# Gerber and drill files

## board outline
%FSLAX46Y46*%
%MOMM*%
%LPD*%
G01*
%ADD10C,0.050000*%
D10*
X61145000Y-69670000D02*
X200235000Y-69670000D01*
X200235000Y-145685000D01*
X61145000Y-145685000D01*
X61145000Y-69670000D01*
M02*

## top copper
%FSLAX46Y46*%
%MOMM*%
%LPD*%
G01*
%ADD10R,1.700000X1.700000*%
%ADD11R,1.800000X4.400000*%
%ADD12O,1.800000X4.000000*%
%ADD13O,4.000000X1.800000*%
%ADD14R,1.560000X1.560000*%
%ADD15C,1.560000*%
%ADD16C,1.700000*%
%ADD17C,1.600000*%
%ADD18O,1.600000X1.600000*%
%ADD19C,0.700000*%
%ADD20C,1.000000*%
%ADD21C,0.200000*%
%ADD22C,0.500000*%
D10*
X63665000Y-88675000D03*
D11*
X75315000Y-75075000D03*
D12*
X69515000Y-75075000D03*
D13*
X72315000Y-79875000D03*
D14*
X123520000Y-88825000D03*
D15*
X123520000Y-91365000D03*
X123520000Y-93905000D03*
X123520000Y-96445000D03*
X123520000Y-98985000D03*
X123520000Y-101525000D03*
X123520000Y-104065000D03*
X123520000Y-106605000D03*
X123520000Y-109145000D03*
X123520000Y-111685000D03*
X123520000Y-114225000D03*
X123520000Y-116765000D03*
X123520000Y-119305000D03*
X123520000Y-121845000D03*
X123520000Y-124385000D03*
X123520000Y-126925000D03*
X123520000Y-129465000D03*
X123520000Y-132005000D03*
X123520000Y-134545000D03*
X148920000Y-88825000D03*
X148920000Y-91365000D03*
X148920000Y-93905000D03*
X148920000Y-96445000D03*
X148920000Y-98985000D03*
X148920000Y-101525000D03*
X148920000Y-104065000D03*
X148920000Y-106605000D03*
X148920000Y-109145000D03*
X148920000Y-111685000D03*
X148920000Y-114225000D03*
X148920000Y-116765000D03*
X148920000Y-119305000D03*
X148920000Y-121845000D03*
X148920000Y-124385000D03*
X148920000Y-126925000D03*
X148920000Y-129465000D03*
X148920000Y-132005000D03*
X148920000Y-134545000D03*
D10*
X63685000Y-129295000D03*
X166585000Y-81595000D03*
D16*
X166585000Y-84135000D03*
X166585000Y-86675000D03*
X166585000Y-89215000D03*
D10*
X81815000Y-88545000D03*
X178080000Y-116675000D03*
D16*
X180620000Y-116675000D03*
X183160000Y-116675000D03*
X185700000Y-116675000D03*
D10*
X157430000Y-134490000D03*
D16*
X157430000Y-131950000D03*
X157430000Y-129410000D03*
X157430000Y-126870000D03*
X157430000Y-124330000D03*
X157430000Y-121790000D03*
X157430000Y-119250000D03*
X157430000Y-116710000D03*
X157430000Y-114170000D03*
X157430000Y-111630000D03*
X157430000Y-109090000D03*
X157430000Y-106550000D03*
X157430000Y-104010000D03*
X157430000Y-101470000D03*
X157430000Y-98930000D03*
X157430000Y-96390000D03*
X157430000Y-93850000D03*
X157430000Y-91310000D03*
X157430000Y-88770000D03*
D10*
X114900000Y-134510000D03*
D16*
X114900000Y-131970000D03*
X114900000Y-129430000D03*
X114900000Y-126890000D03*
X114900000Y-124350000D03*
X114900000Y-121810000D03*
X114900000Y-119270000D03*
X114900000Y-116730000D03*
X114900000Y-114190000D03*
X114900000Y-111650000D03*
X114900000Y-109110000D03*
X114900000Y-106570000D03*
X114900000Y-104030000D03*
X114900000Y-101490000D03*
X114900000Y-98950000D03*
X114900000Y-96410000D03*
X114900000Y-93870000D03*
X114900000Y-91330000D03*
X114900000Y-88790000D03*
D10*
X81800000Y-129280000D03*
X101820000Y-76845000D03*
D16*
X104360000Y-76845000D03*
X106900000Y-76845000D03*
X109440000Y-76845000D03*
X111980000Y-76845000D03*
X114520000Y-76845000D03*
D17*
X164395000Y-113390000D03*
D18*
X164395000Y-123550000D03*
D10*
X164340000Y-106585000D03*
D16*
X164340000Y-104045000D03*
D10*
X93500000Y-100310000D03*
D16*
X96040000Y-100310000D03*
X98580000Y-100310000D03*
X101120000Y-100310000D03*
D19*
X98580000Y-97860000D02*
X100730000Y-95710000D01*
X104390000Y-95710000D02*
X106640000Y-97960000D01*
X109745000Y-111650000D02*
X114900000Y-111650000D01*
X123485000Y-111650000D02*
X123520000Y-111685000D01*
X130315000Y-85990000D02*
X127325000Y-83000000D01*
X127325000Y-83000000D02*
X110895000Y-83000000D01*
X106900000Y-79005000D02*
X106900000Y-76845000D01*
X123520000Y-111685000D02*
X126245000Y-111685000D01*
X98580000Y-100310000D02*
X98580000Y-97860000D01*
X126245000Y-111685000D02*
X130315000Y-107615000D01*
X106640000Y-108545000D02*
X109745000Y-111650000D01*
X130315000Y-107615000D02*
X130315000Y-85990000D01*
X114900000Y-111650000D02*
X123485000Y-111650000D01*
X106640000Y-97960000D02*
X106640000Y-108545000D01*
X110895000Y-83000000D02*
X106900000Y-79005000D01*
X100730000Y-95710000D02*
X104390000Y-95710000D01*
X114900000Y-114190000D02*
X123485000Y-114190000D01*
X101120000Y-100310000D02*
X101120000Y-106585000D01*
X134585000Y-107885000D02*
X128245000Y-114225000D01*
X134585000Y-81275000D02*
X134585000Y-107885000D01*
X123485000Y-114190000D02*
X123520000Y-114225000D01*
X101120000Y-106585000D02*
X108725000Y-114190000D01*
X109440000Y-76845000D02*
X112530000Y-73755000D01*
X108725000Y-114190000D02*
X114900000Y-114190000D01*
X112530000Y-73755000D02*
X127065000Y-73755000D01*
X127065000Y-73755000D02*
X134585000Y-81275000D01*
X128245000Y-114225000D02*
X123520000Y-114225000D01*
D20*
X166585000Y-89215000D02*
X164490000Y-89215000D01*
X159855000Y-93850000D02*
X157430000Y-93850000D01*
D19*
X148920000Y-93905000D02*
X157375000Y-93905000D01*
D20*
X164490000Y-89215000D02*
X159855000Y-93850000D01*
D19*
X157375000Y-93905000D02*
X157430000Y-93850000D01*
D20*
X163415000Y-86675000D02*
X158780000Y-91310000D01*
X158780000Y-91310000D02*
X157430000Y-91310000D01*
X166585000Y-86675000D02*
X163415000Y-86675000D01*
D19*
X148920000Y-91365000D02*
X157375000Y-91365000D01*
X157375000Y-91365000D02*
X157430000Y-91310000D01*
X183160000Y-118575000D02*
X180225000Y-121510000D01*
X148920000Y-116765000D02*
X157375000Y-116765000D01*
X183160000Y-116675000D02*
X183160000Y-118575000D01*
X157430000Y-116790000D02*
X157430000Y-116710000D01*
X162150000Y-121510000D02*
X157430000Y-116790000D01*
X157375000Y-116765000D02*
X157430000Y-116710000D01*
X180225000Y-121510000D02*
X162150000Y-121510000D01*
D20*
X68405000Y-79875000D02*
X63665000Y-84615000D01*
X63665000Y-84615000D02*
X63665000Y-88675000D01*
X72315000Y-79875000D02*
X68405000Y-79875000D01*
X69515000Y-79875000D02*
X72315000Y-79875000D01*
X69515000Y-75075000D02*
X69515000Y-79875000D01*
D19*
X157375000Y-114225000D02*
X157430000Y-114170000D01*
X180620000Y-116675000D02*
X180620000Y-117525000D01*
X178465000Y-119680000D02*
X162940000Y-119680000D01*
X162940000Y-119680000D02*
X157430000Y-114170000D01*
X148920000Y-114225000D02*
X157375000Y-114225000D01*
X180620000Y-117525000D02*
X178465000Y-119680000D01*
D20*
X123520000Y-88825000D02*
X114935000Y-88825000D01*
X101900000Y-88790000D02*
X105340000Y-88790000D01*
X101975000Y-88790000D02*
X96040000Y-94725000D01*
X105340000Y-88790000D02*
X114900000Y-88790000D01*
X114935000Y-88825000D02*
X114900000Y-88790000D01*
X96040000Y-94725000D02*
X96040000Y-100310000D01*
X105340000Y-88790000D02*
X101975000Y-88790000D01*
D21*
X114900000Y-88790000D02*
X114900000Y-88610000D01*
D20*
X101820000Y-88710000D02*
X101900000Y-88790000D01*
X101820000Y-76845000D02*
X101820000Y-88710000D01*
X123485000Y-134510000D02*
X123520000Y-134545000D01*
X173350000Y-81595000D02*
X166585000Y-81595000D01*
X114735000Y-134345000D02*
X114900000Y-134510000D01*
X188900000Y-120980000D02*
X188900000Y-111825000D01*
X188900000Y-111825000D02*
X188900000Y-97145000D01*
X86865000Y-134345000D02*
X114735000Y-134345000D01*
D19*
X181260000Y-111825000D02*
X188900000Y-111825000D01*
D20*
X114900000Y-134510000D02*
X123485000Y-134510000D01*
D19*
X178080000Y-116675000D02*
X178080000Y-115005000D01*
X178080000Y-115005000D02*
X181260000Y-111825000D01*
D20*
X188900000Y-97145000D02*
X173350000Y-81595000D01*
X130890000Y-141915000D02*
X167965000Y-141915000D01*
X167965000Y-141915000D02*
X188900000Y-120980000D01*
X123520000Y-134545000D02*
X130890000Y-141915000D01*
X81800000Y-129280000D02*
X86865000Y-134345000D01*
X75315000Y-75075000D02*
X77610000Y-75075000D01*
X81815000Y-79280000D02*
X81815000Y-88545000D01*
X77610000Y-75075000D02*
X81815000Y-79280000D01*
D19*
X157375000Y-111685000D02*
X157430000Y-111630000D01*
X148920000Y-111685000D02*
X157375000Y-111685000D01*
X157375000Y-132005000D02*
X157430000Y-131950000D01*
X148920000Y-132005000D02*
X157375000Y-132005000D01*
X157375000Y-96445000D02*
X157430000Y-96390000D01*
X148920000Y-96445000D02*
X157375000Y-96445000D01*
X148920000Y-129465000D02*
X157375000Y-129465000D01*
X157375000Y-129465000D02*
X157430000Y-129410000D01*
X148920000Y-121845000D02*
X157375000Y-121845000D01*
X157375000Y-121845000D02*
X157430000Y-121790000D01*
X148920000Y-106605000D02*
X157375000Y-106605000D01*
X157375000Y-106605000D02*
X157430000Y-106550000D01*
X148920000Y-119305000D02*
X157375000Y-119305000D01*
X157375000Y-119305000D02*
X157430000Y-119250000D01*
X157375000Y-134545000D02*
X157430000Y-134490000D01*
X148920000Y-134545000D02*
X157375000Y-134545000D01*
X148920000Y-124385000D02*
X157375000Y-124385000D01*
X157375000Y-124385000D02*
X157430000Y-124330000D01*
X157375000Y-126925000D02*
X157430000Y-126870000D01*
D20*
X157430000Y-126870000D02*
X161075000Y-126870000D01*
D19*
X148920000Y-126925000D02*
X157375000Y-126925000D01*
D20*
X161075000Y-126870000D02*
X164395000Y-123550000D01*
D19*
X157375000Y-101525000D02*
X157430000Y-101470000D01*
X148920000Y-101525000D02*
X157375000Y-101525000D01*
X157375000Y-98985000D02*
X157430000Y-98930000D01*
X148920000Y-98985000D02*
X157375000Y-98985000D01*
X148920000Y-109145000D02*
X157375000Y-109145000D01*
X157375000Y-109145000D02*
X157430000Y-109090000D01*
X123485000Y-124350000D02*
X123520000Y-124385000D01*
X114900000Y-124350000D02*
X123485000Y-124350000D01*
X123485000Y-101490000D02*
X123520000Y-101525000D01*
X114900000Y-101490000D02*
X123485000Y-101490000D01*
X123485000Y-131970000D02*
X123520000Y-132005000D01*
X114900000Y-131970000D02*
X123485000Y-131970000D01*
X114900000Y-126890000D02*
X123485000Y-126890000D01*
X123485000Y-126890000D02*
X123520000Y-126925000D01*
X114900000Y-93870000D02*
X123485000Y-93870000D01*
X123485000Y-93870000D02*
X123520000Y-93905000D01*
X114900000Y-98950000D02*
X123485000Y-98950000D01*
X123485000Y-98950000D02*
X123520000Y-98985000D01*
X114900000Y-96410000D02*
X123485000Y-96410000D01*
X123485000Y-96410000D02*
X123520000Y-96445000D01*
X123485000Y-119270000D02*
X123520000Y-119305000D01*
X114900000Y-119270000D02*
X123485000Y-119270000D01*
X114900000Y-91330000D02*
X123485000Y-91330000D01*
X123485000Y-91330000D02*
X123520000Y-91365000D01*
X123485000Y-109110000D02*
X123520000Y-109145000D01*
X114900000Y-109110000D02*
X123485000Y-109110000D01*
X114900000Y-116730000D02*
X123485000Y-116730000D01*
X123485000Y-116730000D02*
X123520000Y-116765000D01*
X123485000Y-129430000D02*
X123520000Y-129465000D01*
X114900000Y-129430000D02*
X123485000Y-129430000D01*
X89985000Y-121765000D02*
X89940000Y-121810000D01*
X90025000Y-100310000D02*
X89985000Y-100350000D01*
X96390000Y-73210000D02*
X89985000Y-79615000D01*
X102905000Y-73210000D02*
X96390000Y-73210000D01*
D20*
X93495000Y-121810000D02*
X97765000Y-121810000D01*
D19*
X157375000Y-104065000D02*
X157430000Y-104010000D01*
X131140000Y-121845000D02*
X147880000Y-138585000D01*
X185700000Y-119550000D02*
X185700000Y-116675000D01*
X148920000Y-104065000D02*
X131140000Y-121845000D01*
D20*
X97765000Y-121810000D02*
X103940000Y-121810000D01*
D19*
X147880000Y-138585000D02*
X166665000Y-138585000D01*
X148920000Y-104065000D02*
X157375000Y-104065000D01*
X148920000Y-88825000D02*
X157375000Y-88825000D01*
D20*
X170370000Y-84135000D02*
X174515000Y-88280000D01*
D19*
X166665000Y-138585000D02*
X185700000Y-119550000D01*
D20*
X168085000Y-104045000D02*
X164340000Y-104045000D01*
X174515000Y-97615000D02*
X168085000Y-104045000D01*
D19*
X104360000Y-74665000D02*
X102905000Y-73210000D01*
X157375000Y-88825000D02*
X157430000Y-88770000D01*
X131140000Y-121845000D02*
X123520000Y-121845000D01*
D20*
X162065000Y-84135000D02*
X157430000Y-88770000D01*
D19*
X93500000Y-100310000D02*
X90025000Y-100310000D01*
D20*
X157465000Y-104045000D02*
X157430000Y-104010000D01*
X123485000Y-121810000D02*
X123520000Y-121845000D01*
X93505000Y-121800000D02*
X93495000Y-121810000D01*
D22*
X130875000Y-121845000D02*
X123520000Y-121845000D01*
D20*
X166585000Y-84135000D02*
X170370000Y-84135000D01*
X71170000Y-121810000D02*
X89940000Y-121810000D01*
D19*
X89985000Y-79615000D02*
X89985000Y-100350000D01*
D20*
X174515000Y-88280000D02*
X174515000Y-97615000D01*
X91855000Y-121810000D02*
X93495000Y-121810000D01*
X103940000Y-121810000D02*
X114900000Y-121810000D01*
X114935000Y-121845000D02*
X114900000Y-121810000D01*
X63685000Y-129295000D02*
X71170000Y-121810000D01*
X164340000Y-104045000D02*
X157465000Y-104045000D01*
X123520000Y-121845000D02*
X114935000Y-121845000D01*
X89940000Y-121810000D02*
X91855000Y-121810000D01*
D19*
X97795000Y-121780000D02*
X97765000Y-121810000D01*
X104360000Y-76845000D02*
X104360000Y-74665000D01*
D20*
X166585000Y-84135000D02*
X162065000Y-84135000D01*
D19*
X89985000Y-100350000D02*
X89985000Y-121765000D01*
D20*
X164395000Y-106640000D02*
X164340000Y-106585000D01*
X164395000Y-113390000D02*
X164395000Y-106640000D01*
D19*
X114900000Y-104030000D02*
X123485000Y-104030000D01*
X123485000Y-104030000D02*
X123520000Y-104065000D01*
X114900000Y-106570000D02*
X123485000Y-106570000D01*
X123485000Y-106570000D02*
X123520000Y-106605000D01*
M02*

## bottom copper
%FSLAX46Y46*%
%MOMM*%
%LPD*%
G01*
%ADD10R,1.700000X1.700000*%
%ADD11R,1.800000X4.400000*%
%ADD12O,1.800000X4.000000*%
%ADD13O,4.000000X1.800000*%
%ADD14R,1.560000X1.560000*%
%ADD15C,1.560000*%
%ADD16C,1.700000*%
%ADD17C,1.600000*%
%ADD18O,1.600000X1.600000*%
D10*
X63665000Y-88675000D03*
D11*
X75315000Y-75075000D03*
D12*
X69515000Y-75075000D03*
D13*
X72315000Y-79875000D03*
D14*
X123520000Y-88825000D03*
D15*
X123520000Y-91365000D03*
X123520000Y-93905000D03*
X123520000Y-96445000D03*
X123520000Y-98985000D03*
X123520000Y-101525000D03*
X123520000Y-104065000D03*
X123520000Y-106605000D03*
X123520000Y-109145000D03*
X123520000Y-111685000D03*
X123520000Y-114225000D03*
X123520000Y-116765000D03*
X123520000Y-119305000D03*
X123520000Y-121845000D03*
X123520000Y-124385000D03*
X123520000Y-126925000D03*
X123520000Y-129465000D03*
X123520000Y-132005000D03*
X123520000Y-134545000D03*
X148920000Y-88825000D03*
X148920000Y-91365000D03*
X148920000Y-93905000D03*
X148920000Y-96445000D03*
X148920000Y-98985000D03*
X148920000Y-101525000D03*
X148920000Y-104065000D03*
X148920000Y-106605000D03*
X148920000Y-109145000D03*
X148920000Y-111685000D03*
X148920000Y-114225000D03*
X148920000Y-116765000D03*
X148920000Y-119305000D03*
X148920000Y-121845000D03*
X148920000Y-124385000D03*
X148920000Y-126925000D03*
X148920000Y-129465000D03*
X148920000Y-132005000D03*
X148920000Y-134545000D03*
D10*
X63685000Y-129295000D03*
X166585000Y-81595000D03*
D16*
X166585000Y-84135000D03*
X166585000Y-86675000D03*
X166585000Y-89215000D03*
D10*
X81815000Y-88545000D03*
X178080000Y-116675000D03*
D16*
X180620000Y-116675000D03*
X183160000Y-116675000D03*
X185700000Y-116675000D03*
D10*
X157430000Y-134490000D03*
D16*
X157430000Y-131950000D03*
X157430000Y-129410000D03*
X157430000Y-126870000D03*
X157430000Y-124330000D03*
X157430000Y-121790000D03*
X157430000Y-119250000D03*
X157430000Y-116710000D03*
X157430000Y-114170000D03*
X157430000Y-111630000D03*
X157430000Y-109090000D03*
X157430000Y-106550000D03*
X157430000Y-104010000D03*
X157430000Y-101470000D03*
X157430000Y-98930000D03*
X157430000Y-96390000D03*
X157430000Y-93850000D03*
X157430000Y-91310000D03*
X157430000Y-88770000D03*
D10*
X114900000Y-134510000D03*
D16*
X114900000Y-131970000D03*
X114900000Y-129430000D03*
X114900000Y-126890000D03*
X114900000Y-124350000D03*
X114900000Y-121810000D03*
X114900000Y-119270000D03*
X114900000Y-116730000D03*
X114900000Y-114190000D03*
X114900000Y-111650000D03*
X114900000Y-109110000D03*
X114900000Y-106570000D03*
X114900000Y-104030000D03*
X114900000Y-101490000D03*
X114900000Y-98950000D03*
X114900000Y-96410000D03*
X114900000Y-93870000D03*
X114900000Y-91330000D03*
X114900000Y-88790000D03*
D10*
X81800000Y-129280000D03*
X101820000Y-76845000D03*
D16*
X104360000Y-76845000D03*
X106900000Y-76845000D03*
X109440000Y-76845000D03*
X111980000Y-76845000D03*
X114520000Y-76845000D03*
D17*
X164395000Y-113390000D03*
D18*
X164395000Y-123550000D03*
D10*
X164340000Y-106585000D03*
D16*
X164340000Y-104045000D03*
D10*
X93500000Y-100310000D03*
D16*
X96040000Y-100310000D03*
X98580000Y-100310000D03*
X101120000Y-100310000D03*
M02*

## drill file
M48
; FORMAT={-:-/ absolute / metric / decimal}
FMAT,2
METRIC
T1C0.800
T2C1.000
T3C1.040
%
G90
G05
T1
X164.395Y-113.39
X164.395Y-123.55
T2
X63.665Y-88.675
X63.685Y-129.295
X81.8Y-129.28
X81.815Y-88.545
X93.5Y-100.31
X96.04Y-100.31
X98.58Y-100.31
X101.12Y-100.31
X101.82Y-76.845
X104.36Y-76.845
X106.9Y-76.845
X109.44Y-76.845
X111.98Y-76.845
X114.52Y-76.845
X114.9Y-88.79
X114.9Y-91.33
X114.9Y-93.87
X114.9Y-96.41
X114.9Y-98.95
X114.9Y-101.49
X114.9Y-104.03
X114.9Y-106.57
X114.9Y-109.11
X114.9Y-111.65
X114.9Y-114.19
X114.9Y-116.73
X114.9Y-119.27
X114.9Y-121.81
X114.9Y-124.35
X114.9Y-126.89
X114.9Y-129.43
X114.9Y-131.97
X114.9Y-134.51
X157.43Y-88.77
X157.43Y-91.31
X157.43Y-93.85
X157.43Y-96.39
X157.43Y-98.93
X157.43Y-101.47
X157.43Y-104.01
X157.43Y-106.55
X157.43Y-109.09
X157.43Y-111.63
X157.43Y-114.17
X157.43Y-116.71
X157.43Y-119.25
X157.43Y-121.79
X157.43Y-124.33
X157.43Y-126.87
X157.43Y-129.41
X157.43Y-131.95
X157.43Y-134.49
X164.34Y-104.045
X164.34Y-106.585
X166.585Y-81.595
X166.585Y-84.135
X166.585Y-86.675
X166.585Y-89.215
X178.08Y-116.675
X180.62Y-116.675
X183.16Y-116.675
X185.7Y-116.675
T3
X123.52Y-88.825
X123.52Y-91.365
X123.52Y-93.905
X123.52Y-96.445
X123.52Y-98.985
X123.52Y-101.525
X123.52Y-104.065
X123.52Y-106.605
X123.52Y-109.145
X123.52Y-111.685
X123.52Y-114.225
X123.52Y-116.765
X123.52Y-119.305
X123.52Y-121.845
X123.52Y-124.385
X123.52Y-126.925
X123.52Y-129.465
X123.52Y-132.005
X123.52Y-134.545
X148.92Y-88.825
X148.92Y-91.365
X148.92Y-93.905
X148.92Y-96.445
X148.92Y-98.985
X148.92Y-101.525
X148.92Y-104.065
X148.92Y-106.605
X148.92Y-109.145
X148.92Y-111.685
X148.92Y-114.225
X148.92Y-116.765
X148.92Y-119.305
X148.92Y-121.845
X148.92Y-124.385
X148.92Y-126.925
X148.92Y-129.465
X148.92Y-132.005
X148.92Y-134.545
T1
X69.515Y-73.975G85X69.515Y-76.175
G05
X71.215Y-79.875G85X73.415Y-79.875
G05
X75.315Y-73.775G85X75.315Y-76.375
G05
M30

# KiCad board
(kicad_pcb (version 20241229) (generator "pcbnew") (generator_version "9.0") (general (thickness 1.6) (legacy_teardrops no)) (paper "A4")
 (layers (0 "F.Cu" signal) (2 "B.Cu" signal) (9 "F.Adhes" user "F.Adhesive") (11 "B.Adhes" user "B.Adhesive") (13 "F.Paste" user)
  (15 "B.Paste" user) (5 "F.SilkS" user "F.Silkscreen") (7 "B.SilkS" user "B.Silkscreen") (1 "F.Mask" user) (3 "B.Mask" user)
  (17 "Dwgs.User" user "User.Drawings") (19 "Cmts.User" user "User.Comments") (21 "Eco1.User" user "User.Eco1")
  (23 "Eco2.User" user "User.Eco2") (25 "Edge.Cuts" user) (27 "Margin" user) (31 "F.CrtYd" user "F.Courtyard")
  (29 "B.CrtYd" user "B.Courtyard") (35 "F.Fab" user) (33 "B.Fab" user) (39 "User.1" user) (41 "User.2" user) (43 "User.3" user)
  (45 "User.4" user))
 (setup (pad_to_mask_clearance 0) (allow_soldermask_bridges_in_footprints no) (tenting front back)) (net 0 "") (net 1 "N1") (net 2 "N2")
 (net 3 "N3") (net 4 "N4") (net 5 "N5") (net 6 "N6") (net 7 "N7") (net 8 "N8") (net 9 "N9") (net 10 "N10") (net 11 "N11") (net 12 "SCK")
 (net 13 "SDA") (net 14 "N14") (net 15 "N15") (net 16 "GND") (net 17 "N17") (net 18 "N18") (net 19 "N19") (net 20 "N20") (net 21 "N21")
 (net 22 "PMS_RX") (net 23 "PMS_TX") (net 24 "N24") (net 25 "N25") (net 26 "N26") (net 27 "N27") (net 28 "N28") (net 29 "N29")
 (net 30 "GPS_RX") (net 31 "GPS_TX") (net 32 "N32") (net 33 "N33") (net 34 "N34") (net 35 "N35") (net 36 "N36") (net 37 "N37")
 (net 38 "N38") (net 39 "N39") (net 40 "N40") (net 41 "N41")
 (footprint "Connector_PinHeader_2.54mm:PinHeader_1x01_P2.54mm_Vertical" (layer "F.Cu") (at 63.665 88.675)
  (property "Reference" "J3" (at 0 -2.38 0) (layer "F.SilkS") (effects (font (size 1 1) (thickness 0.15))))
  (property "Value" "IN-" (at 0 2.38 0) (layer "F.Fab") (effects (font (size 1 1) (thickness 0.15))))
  (pad "1" thru_hole rect (at 0 0) (size 1.7 1.7) (drill 1) (layers "*.Cu" "*.Mask") (remove_unused_layers no) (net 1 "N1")))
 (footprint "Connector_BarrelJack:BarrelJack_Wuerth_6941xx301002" (layer "F.Cu") (at 75.315 75.075 -90)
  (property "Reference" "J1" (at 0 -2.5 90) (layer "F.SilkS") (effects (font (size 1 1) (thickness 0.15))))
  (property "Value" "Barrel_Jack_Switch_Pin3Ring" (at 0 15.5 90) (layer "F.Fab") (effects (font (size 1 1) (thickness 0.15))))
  (pad "1" thru_hole rect (at 0 0 270) (size 4.4 1.8) (drill oval 3.4 0.8) (layers "*.Cu" "*.Mask") (remove_unused_layers no) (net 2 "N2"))
  (pad "2" thru_hole oval (at 0 5.8 270) (size 4 1.8) (drill oval 3 0.8) (layers "*.Cu" "*.Mask") (remove_unused_layers no) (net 1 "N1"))
  (pad "3" thru_hole oval (at 4.8 3) (size 4 1.8) (drill oval 3 0.8) (layers "*.Cu" "*.Mask") (remove_unused_layers no) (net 1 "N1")))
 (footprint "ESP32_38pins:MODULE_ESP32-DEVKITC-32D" (layer "F.Cu") (at 136.22 108.585)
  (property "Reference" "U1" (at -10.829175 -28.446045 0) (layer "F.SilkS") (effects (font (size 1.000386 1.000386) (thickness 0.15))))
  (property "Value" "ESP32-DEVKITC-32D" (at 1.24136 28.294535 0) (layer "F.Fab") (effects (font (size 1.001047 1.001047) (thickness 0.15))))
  (pad "J2-1" thru_hole rect (at -12.7 -19.76) (size 1.56 1.56) (drill 1.04) (layers "*.Cu" "*.Mask") (remove_unused_layers no) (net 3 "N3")
   (solder_mask_margin 0.102))
  (pad "J2-2" thru_hole circle (at -12.7 -17.22) (size 1.56 1.56) (drill 1.04) (layers "*.Cu" "*.Mask") (remove_unused_layers no)
   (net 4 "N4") (solder_mask_margin 0.102))
  (pad "J2-3" thru_hole circle (at -12.7 -14.68) (size 1.56 1.56) (drill 1.04) (layers "*.Cu" "*.Mask") (remove_unused_layers no)
   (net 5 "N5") (solder_mask_margin 0.102))
  (pad "J2-4" thru_hole circle (at -12.7 -12.14) (size 1.56 1.56) (drill 1.04) (layers "*.Cu" "*.Mask") (remove_unused_layers no)
   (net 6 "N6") (solder_mask_margin 0.102))
  (pad "J2-5" thru_hole circle (at -12.7 -9.6) (size 1.56 1.56) (drill 1.04) (layers "*.Cu" "*.Mask") (remove_unused_layers no) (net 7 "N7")
   (solder_mask_margin 0.102))
  (pad "J2-6" thru_hole circle (at -12.7 -7.06) (size 1.56 1.56) (drill 1.04) (layers "*.Cu" "*.Mask") (remove_unused_layers no)
   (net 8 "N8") (solder_mask_margin 0.102))
  (pad "J2-7" thru_hole circle (at -12.7 -4.52) (size 1.56 1.56) (drill 1.04) (layers "*.Cu" "*.Mask") (remove_unused_layers no)
   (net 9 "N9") (solder_mask_margin 0.102))
  (pad "J2-8" thru_hole circle (at -12.7 -1.98) (size 1.56 1.56) (drill 1.04) (layers "*.Cu" "*.Mask") (remove_unused_layers no)
   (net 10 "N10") (solder_mask_margin 0.102))
  (pad "J2-9" thru_hole circle (at -12.7 0.56) (size 1.56 1.56) (drill 1.04) (layers "*.Cu" "*.Mask") (remove_unused_layers no)
   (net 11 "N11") (solder_mask_margin 0.102))
  (pad "J2-10" thru_hole circle (at -12.7 3.1) (size 1.56 1.56) (drill 1.04) (layers "*.Cu" "*.Mask") (remove_unused_layers no)
   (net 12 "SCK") (solder_mask_margin 0.102))
  (pad "J2-11" thru_hole circle (at -12.7 5.64) (size 1.56 1.56) (drill 1.04) (layers "*.Cu" "*.Mask") (remove_unused_layers no)
   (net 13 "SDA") (solder_mask_margin 0.102))
  (pad "J2-12" thru_hole circle (at -12.7 8.18) (size 1.56 1.56) (drill 1.04) (layers "*.Cu" "*.Mask") (remove_unused_layers no)
   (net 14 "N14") (solder_mask_margin 0.102))
  (pad "J2-13" thru_hole circle (at -12.7 10.72) (size 1.56 1.56) (drill 1.04) (layers "*.Cu" "*.Mask") (remove_unused_layers no)
   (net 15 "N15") (solder_mask_margin 0.102))
  (pad "J2-14" thru_hole circle (at -12.7 13.26) (size 1.56 1.56) (drill 1.04) (layers "*.Cu" "*.Mask") (remove_unused_layers no)
   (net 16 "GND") (solder_mask_margin 0.102))
  (pad "J2-15" thru_hole circle (at -12.7 15.8) (size 1.56 1.56) (drill 1.04) (layers "*.Cu" "*.Mask") (remove_unused_layers no)
   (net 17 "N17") (solder_mask_margin 0.102))
  (pad "J2-16" thru_hole circle (at -12.7 18.34) (size 1.56 1.56) (drill 1.04) (layers "*.Cu" "*.Mask") (remove_unused_layers no)
   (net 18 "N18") (solder_mask_margin 0.102))
  (pad "J2-17" thru_hole circle (at -12.7 20.88) (size 1.56 1.56) (drill 1.04) (layers "*.Cu" "*.Mask") (remove_unused_layers no)
   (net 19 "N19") (solder_mask_margin 0.102))
  (pad "J2-18" thru_hole circle (at -12.7 23.42) (size 1.56 1.56) (drill 1.04) (layers "*.Cu" "*.Mask") (remove_unused_layers no)
   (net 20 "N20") (solder_mask_margin 0.102))
  (pad "J2-19" thru_hole circle (at -12.7 25.96) (size 1.56 1.56) (drill 1.04) (layers "*.Cu" "*.Mask") (remove_unused_layers no)
   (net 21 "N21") (solder_mask_margin 0.102))
  (pad "J3-1" thru_hole circle (at 12.7 -19.76) (size 1.56 1.56) (drill 1.04) (layers "*.Cu" "*.Mask") (remove_unused_layers no)
   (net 16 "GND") (solder_mask_margin 0.102))
  (pad "J3-2" thru_hole circle (at 12.7 -17.22) (size 1.56 1.56) (drill 1.04) (layers "*.Cu" "*.Mask") (remove_unused_layers no)
   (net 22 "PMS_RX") (solder_mask_margin 0.102))
  (pad "J3-3" thru_hole circle (at 12.7 -14.68) (size 1.56 1.56) (drill 1.04) (layers "*.Cu" "*.Mask") (remove_unused_layers no)
   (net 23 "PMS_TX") (solder_mask_margin 0.102))
  (pad "J3-4" thru_hole circle (at 12.7 -12.14) (size 1.56 1.56) (drill 1.04) (layers "*.Cu" "*.Mask") (remove_unused_layers no)
   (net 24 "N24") (solder_mask_margin 0.102))
  (pad "J3-5" thru_hole circle (at 12.7 -9.6) (size 1.56 1.56) (drill 1.04) (layers "*.Cu" "*.Mask") (remove_unused_layers no)
   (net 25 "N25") (solder_mask_margin 0.102))
  (pad "J3-6" thru_hole circle (at 12.7 -7.06) (size 1.56 1.56) (drill 1.04) (layers "*.Cu" "*.Mask") (remove_unused_layers no)
   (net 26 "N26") (solder_mask_margin 0.102))
  (pad "J3-7" thru_hole circle (at 12.7 -4.52) (size 1.56 1.56) (drill 1.04) (layers "*.Cu" "*.Mask") (remove_unused_layers no)
   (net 16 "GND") (solder_mask_margin 0.102))
  (pad "J3-8" thru_hole circle (at 12.7 -1.98) (size 1.56 1.56) (drill 1.04) (layers "*.Cu" "*.Mask") (remove_unused_layers no)
   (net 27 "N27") (solder_mask_margin 0.102))
  (pad "J3-9" thru_hole circle (at 12.7 0.56) (size 1.56 1.56) (drill 1.04) (layers "*.Cu" "*.Mask") (remove_unused_layers no)
   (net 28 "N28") (solder_mask_margin 0.102))
  (pad "J3-10" thru_hole circle (at 12.7 3.1) (size 1.56 1.56) (drill 1.04) (layers "*.Cu" "*.Mask") (remove_unused_layers no)
   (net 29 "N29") (solder_mask_margin 0.102))
  (pad "J3-11" thru_hole circle (at 12.7 5.64) (size 1.56 1.56) (drill 1.04) (layers "*.Cu" "*.Mask") (remove_unused_layers no)
   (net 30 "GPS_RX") (solder_mask_margin 0.102))
  (pad "J3-12" thru_hole circle (at 12.7 8.18) (size 1.56 1.56) (drill 1.04) (layers "*.Cu" "*.Mask") (remove_unused_layers no)
   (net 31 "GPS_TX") (solder_mask_margin 0.102))
  (pad "J3-13" thru_hole circle (at 12.7 10.72) (size 1.56 1.56) (drill 1.04) (layers "*.Cu" "*.Mask") (remove_unused_layers no)
   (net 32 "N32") (solder_mask_margin 0.102))
  (pad "J3-14" thru_hole circle (at 12.7 13.26) (size 1.56 1.56) (drill 1.04) (layers "*.Cu" "*.Mask") (remove_unused_layers no)
   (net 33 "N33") (solder_mask_margin 0.102))
  (pad "J3-15" thru_hole circle (at 12.7 15.8) (size 1.56 1.56) (drill 1.04) (layers "*.Cu" "*.Mask") (remove_unused_layers no)
   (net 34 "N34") (solder_mask_margin 0.102))
  (pad "J3-16" thru_hole circle (at 12.7 18.34) (size 1.56 1.56) (drill 1.04) (layers "*.Cu" "*.Mask") (remove_unused_layers no)
   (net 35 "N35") (solder_mask_margin 0.102))
  (pad "J3-17" thru_hole circle (at 12.7 20.88) (size 1.56 1.56) (drill 1.04) (layers "*.Cu" "*.Mask") (remove_unused_layers no)
   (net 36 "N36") (solder_mask_margin 0.102))
  (pad "J3-18" thru_hole circle (at 12.7 23.42) (size 1.56 1.56) (drill 1.04) (layers "*.Cu" "*.Mask") (remove_unused_layers no)
   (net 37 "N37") (solder_mask_margin 0.102))
  (pad "J3-19" thru_hole circle (at 12.7 25.96) (size 1.56 1.56) (drill 1.04) (layers "*.Cu" "*.Mask") (remove_unused_layers no)
   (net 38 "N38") (solder_mask_margin 0.102)))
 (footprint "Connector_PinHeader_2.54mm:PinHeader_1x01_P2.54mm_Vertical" (layer "F.Cu") (at 63.685 129.295)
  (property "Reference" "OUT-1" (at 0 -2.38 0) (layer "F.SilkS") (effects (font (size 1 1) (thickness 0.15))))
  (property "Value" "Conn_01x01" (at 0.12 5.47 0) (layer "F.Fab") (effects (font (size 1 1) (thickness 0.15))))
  (pad "1" thru_hole rect (at 0 0) (size 1.7 1.7) (drill 1) (layers "*.Cu" "*.Mask") (remove_unused_layers no) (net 16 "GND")))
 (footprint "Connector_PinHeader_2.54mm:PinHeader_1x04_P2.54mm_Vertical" (layer "F.Cu") (at 166.585 81.595)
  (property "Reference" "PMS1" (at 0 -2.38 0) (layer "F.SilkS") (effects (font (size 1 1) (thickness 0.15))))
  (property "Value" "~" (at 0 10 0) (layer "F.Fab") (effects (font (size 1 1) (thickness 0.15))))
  (pad "1" thru_hole rect (at 0 0) (size 1.7 1.7) (drill 1) (layers "*.Cu" "*.Mask") (remove_unused_layers no) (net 21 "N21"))
  (pad "2" thru_hole circle (at 0 2.54) (size 1.7 1.7) (drill 1) (layers "*.Cu" "*.Mask") (remove_unused_layers no) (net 16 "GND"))
  (pad "3" thru_hole circle (at 0 5.08) (size 1.7 1.7) (drill 1) (layers "*.Cu" "*.Mask") (remove_unused_layers no) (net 22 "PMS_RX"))
  (pad "4" thru_hole circle (at 0 7.62) (size 1.7 1.7) (drill 1) (layers "*.Cu" "*.Mask") (remove_unused_layers no) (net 23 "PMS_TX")))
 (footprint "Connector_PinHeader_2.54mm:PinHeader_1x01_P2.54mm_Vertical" (layer "F.Cu") (at 81.815 88.545)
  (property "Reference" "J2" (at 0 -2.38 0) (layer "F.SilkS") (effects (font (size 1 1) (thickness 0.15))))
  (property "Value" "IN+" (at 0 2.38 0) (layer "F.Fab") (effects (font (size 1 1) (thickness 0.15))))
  (pad "1" thru_hole rect (at 0 0) (size 1.7 1.7) (drill 1) (layers "*.Cu" "*.Mask") (remove_unused_layers no) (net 2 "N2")))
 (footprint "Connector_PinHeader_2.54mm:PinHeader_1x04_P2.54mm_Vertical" (layer "F.Cu") (at 178.08 116.675 90)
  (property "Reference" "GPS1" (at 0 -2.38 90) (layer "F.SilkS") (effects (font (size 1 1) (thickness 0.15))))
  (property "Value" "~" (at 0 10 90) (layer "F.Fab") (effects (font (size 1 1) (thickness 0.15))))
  (pad "1" thru_hole rect (at 0 0 90) (size 1.7 1.7) (drill 1) (layers "*.Cu" "*.Mask") (remove_unused_layers no) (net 21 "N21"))
  (pad "2" thru_hole circle (at 0 2.54 90) (size 1.7 1.7) (drill 1) (layers "*.Cu" "*.Mask") (remove_unused_layers no) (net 30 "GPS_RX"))
  (pad "3" thru_hole circle (at 0 5.08 90) (size 1.7 1.7) (drill 1) (layers "*.Cu" "*.Mask") (remove_unused_layers no) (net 31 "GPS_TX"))
  (pad "4" thru_hole circle (at 0 7.62 90) (size 1.7 1.7) (drill 1) (layers "*.Cu" "*.Mask") (remove_unused_layers no) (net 16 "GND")))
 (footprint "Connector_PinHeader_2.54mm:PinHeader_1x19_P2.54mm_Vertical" (layer "F.Cu") (at 157.43 134.49 180)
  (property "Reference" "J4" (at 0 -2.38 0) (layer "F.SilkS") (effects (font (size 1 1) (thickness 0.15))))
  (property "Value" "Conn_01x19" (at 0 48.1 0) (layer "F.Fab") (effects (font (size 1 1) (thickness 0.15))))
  (pad "1" thru_hole rect (at 0 0 180) (size 1.7 1.7) (drill 1) (layers "*.Cu" "*.Mask") (remove_unused_layers no) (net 38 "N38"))
  (pad "2" thru_hole circle (at 0 2.54 180) (size 1.7 1.7) (drill 1) (layers "*.Cu" "*.Mask") (remove_unused_layers no) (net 37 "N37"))
  (pad "3" thru_hole circle (at 0 5.08 180) (size 1.7 1.7) (drill 1) (layers "*.Cu" "*.Mask") (remove_unused_layers no) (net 36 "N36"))
  (pad "4" thru_hole circle (at 0 7.62 180) (size 1.7 1.7) (drill 1) (layers "*.Cu" "*.Mask") (remove_unused_layers no) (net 35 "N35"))
  (pad "5" thru_hole circle (at 0 10.16 180) (size 1.7 1.7) (drill 1) (layers "*.Cu" "*.Mask") (remove_unused_layers no) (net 34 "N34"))
  (pad "6" thru_hole circle (at 0 12.7 180) (size 1.7 1.7) (drill 1) (layers "*.Cu" "*.Mask") (remove_unused_layers no) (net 33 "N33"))
  (pad "7" thru_hole circle (at 0 15.24 180) (size 1.7 1.7) (drill 1) (layers "*.Cu" "*.Mask") (remove_unused_layers no) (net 32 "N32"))
  (pad "8" thru_hole circle (at 0 17.78 180) (size 1.7 1.7) (drill 1) (layers "*.Cu" "*.Mask") (remove_unused_layers no) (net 31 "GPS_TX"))
  (pad "9" thru_hole circle (at 0 20.32 180) (size 1.7 1.7) (drill 1) (layers "*.Cu" "*.Mask") (remove_unused_layers no) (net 30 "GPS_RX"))
  (pad "10" thru_hole circle (at 0 22.86 180) (size 1.7 1.7) (drill 1) (layers "*.Cu" "*.Mask") (remove_unused_layers no) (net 29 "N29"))
  (pad "11" thru_hole circle (at 0 25.4 180) (size 1.7 1.7) (drill 1) (layers "*.Cu" "*.Mask") (remove_unused_layers no) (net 28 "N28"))
  (pad "12" thru_hole circle (at 0 27.94 180) (size 1.7 1.7) (drill 1) (layers "*.Cu" "*.Mask") (remove_unused_layers no) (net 27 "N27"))
  (pad "13" thru_hole circle (at 0 30.48 180) (size 1.7 1.7) (drill 1) (layers "*.Cu" "*.Mask") (remove_unused_layers no) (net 16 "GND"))
  (pad "14" thru_hole circle (at 0 33.02 180) (size 1.7 1.7) (drill 1) (layers "*.Cu" "*.Mask") (remove_unused_layers no) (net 26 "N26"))
  (pad "15" thru_hole circle (at 0 35.56 180) (size 1.7 1.7) (drill 1) (layers "*.Cu" "*.Mask") (remove_unused_layers no) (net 25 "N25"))
  (pad "16" thru_hole circle (at 0 38.1 180) (size 1.7 1.7) (drill 1) (layers "*.Cu" "*.Mask") (remove_unused_layers no) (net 24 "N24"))
  (pad "17" thru_hole circle (at 0 40.64 180) (size 1.7 1.7) (drill 1) (layers "*.Cu" "*.Mask") (remove_unused_layers no) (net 23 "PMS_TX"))
  (pad "18" thru_hole circle (at 0 43.18 180) (size 1.7 1.7) (drill 1) (layers "*.Cu" "*.Mask") (remove_unused_layers no) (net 22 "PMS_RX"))
  (pad "19" thru_hole circle (at 0 45.72 180) (size 1.7 1.7) (drill 1) (layers "*.Cu" "*.Mask") (remove_unused_layers no) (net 16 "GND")))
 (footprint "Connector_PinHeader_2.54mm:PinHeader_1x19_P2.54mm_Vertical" (layer "F.Cu") (at 114.9 134.51 180)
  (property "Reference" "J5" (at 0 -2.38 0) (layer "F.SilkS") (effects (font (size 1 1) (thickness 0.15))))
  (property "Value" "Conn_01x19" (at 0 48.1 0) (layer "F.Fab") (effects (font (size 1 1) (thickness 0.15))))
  (pad "1" thru_hole rect (at 0 0 180) (size 1.7 1.7) (drill 1) (layers "*.Cu" "*.Mask") (remove_unused_layers no) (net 21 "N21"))
  (pad "2" thru_hole circle (at 0 2.54 180) (size 1.7 1.7) (drill 1) (layers "*.Cu" "*.Mask") (remove_unused_layers no) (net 20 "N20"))
  (pad "3" thru_hole circle (at 0 5.08 180) (size 1.7 1.7) (drill 1) (layers "*.Cu" "*.Mask") (remove_unused_layers no) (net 19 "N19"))
  (pad "4" thru_hole circle (at 0 7.62 180) (size 1.7 1.7) (drill 1) (layers "*.Cu" "*.Mask") (remove_unused_layers no) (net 18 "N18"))
  (pad "5" thru_hole circle (at 0 10.16 180) (size 1.7 1.7) (drill 1) (layers "*.Cu" "*.Mask") (remove_unused_layers no) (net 17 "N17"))
  (pad "6" thru_hole circle (at 0 12.7 180) (size 1.7 1.7) (drill 1) (layers "*.Cu" "*.Mask") (remove_unused_layers no) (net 16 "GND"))
  (pad "7" thru_hole circle (at 0 15.24 180) (size 1.7 1.7) (drill 1) (layers "*.Cu" "*.Mask") (remove_unused_layers no) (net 15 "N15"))
  (pad "8" thru_hole circle (at 0 17.78 180) (size 1.7 1.7) (drill 1) (layers "*.Cu" "*.Mask") (remove_unused_layers no) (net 14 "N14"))
  (pad "9" thru_hole circle (at 0 20.32 180) (size 1.7 1.7) (drill 1) (layers "*.Cu" "*.Mask") (remove_unused_layers no) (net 13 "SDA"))
  (pad "10" thru_hole circle (at 0 22.86 180) (size 1.7 1.7) (drill 1) (layers "*.Cu" "*.Mask") (remove_unused_layers no) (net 12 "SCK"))
  (pad "11" thru_hole circle (at 0 25.4 180) (size 1.7 1.7) (drill 1) (layers "*.Cu" "*.Mask") (remove_unused_layers no) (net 11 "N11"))
  (pad "12" thru_hole circle (at 0 27.94 180) (size 1.7 1.7) (drill 1) (layers "*.Cu" "*.Mask") (remove_unused_layers no) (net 10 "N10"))
  (pad "13" thru_hole circle (at 0 30.48 180) (size 1.7 1.7) (drill 1) (layers "*.Cu" "*.Mask") (remove_unused_layers no) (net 9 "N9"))
  (pad "14" thru_hole circle (at 0 33.02 180) (size 1.7 1.7) (drill 1) (layers "*.Cu" "*.Mask") (remove_unused_layers no) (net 8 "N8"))
  (pad "15" thru_hole circle (at 0 35.56 180) (size 1.7 1.7) (drill 1) (layers "*.Cu" "*.Mask") (remove_unused_layers no) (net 7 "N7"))
  (pad "16" thru_hole circle (at 0 38.1 180) (size 1.7 1.7) (drill 1) (layers "*.Cu" "*.Mask") (remove_unused_layers no) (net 6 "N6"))
  (pad "17" thru_hole circle (at 0 40.64 180) (size 1.7 1.7) (drill 1) (layers "*.Cu" "*.Mask") (remove_unused_layers no) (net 5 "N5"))
  (pad "18" thru_hole circle (at 0 43.18 180) (size 1.7 1.7) (drill 1) (layers "*.Cu" "*.Mask") (remove_unused_layers no) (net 4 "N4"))
  (pad "19" thru_hole circle (at 0 45.72 180) (size 1.7 1.7) (drill 1) (layers "*.Cu" "*.Mask") (remove_unused_layers no) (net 3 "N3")))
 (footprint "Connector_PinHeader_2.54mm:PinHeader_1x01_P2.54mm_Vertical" (layer "F.Cu") (at 81.8 129.28)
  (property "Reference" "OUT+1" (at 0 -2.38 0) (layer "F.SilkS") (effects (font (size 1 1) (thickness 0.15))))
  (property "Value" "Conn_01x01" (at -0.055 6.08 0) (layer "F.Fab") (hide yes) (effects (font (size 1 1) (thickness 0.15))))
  (pad "1" thru_hole rect (at 0 0) (size 1.7 1.7) (drill 1) (layers "*.Cu" "*.Mask") (remove_unused_layers no) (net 21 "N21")))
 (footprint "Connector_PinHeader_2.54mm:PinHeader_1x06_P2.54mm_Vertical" (layer "F.Cu") (at 101.82 76.845 90)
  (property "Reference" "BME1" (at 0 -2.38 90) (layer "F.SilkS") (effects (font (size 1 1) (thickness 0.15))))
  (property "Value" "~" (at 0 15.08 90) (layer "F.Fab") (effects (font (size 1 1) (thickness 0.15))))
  (pad "1" thru_hole rect (at 0 0 90) (size 1.7 1.7) (drill 1) (layers "*.Cu" "*.Mask") (remove_unused_layers no) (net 3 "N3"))
  (pad "2" thru_hole circle (at 0 2.54 90) (size 1.7 1.7) (drill 1) (layers "*.Cu" "*.Mask") (remove_unused_layers no) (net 16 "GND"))
  (pad "3" thru_hole circle (at 0 5.08 90) (size 1.7 1.7) (drill 1) (layers "*.Cu" "*.Mask") (remove_unused_layers no) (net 12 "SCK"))
  (pad "4" thru_hole circle (at 0 7.62 90) (size 1.7 1.7) (drill 1) (layers "*.Cu" "*.Mask") (remove_unused_layers no) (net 13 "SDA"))
  (pad "5" thru_hole circle (at 0 10.16 90) (size 1.7 1.7) (drill 1) (layers "*.Cu" "*.Mask") (remove_unused_layers no) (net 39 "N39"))
  (pad "6" thru_hole circle (at 0 12.7 90) (size 1.7 1.7) (drill 1) (layers "*.Cu" "*.Mask") (remove_unused_layers no) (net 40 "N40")))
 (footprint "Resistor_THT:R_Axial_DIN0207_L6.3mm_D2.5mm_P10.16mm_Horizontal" (layer "F.Cu") (at 164.395 113.39 -90)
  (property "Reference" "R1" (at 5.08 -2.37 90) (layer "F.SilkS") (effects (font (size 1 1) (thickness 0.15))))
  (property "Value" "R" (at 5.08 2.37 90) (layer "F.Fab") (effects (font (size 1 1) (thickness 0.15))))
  (pad "1" thru_hole circle (at 0 0 270) (size 1.6 1.6) (drill 0.8) (layers "*.Cu" "*.Mask") (remove_unused_layers no) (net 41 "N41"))
  (pad "2" thru_hole oval (at 10.16 0 270) (size 1.6 1.6) (drill 0.8) (layers "*.Cu" "*.Mask") (remove_unused_layers no) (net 35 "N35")))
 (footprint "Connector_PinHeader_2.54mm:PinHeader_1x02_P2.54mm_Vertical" (layer "F.Cu") (at 164.34 106.585 180)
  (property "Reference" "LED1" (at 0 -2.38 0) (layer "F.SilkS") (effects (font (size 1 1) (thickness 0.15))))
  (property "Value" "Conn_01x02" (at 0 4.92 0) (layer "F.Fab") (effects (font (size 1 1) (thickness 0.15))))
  (pad "1" thru_hole rect (at 0 0 180) (size 1.7 1.7) (drill 1) (layers "*.Cu" "*.Mask") (remove_unused_layers no) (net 41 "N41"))
  (pad "2" thru_hole circle (at 0 2.54 180) (size 1.7 1.7) (drill 1) (layers "*.Cu" "*.Mask") (remove_unused_layers no) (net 16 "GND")))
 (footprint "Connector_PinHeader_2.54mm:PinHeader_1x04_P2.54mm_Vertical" (layer "F.Cu") (at 93.5 100.31 90)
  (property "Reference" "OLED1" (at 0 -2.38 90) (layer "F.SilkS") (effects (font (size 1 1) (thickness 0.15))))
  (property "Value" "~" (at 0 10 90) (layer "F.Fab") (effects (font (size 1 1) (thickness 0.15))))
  (pad "1" thru_hole rect (at 0 0 90) (size 1.7 1.7) (drill 1) (layers "*.Cu" "*.Mask") (remove_unused_layers no) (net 16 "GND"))
  (pad "2" thru_hole circle (at 0 2.54 90) (size 1.7 1.7) (drill 1) (layers "*.Cu" "*.Mask") (remove_unused_layers no) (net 3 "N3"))
  (pad "3" thru_hole circle (at 0 5.08 90) (size 1.7 1.7) (drill 1) (layers "*.Cu" "*.Mask") (remove_unused_layers no) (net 12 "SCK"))
  (pad "4" thru_hole circle (at 0 7.62 90) (size 1.7 1.7) (drill 1) (layers "*.Cu" "*.Mask") (remove_unused_layers no) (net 13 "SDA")))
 (gr_rect (start 61.145 69.67) (end 200.235 145.685) (stroke (width 0.05) (type default)) (fill no) (layer "Edge.Cuts"))
 (segment (start 98.58 97.86) (end 100.73 95.71) (width 0.7) (layer "F.Cu") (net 12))
 (segment (start 104.39 95.71) (end 106.64 97.96) (width 0.7) (layer "F.Cu") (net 12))
 (segment (start 109.745 111.65) (end 114.9 111.65) (width 0.7) (layer "F.Cu") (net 12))
 (segment (start 123.485 111.65) (end 123.52 111.685) (width 0.7) (layer "F.Cu") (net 12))
 (segment (start 130.315 85.99) (end 127.325 83) (width 0.7) (layer "F.Cu") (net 12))
 (segment (start 127.325 83) (end 110.895 83) (width 0.7) (layer "F.Cu") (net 12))
 (segment (start 106.9 79.005) (end 106.9 76.845) (width 0.7) (layer "F.Cu") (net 12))
 (segment (start 123.52 111.685) (end 126.245 111.685) (width 0.7) (layer "F.Cu") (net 12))
 (segment (start 98.58 100.31) (end 98.58 97.86) (width 0.7) (layer "F.Cu") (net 12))
 (segment (start 126.245 111.685) (end 130.315 107.615) (width 0.7) (layer "F.Cu") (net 12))
 (segment (start 106.64 108.545) (end 109.745 111.65) (width 0.7) (layer "F.Cu") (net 12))
 (segment (start 130.315 107.615) (end 130.315 85.99) (width 0.7) (layer "F.Cu") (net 12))
 (segment (start 114.9 111.65) (end 123.485 111.65) (width 0.7) (layer "F.Cu") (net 12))
 (segment (start 106.64 97.96) (end 106.64 108.545) (width 0.7) (layer "F.Cu") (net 12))
 (segment (start 110.895 83) (end 106.9 79.005) (width 0.7) (layer "F.Cu") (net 12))
 (segment (start 100.73 95.71) (end 104.39 95.71) (width 0.7) (layer "F.Cu") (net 12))
 (segment (start 114.9 114.19) (end 123.485 114.19) (width 0.7) (layer "F.Cu") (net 13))
 (segment (start 101.12 100.31) (end 101.12 106.585) (width 0.7) (layer "F.Cu") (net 13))
 (segment (start 134.585 107.885) (end 128.245 114.225) (width 0.7) (layer "F.Cu") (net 13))
 (segment (start 134.585 81.275) (end 134.585 107.885) (width 0.7) (layer "F.Cu") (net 13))
 (segment (start 123.485 114.19) (end 123.52 114.225) (width 0.7) (layer "F.Cu") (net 13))
 (segment (start 101.12 106.585) (end 108.725 114.19) (width 0.7) (layer "F.Cu") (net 13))
 (segment (start 109.44 76.845) (end 112.53 73.755) (width 0.7) (layer "F.Cu") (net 13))
 (segment (start 108.725 114.19) (end 114.9 114.19) (width 0.7) (layer "F.Cu") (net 13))
 (segment (start 112.53 73.755) (end 127.065 73.755) (width 0.7) (layer "F.Cu") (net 13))
 (segment (start 127.065 73.755) (end 134.585 81.275) (width 0.7) (layer "F.Cu") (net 13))
 (segment (start 128.245 114.225) (end 123.52 114.225) (width 0.7) (layer "F.Cu") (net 13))
 (segment (start 166.585 89.215) (end 164.49 89.215) (width 1) (layer "F.Cu") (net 23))
 (segment (start 159.855 93.85) (end 157.43 93.85) (width 1) (layer "F.Cu") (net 23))
 (segment (start 148.92 93.905) (end 157.375 93.905) (width 0.7) (layer "F.Cu") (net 23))
 (segment (start 164.49 89.215) (end 159.855 93.85) (width 1) (layer "F.Cu") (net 23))
 (segment (start 157.375 93.905) (end 157.43 93.85) (width 0.7) (layer "F.Cu") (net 23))
 (segment (start 163.415 86.675) (end 158.78 91.31) (width 1) (layer "F.Cu") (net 22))
 (segment (start 158.78 91.31) (end 157.43 91.31) (width 1) (layer "F.Cu") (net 22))
 (segment (start 166.585 86.675) (end 163.415 86.675) (width 1) (layer "F.Cu") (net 22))
 (segment (start 148.92 91.365) (end 157.375 91.365) (width 0.7) (layer "F.Cu") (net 22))
 (segment (start 157.375 91.365) (end 157.43 91.31) (width 0.7) (layer "F.Cu") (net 22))
 (segment (start 183.16 118.575) (end 180.225 121.51) (width 0.7) (layer "F.Cu") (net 31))
 (segment (start 148.92 116.765) (end 157.375 116.765) (width 0.7) (layer "F.Cu") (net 31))
 (segment (start 183.16 116.675) (end 183.16 118.575) (width 0.7) (layer "F.Cu") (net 31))
 (segment (start 157.43 116.79) (end 157.43 116.71) (width 0.7) (layer "F.Cu") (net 31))
 (segment (start 162.15 121.51) (end 157.43 116.79) (width 0.7) (layer "F.Cu") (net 31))
 (segment (start 157.375 116.765) (end 157.43 116.71) (width 0.7) (layer "F.Cu") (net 31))
 (segment (start 180.225 121.51) (end 162.15 121.51) (width 0.7) (layer "F.Cu") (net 31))
 (segment (start 68.405 79.875) (end 63.665 84.615) (width 1) (layer "F.Cu") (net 1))
 (segment (start 63.665 84.615) (end 63.665 88.675) (width 1) (layer "F.Cu") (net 1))
 (segment (start 72.315 79.875) (end 68.405 79.875) (width 1) (layer "F.Cu") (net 1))
 (segment (start 69.515 79.875) (end 72.315 79.875) (width 1) (layer "F.Cu") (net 1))
 (segment (start 69.515 75.075) (end 69.515 79.875) (width 1) (layer "F.Cu") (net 1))
 (segment (start 157.375 114.225) (end 157.43 114.17) (width 0.7) (layer "F.Cu") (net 30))
 (segment (start 180.62 116.675) (end 180.62 117.525) (width 0.7) (layer "F.Cu") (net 30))
 (segment (start 178.465 119.68) (end 162.94 119.68) (width 0.7) (layer "F.Cu") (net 30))
 (segment (start 162.94 119.68) (end 157.43 114.17) (width 0.7) (layer "F.Cu") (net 30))
 (segment (start 148.92 114.225) (end 157.375 114.225) (width 0.7) (layer "F.Cu") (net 30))
 (segment (start 180.62 117.525) (end 178.465 119.68) (width 0.7) (layer "F.Cu") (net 30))
 (segment (start 123.52 88.825) (end 114.935 88.825) (width 1) (layer "F.Cu") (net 3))
 (segment (start 101.9 88.79) (end 105.34 88.79) (width 1) (layer "F.Cu") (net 3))
 (segment (start 101.975 88.79) (end 96.04 94.725) (width 1) (layer "F.Cu") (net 3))
 (segment (start 105.34 88.79) (end 114.9 88.79) (width 1) (layer "F.Cu") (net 3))
 (segment (start 114.935 88.825) (end 114.9 88.79) (width 1) (layer "F.Cu") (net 3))
 (segment (start 96.04 94.725) (end 96.04 100.31) (width 1) (layer "F.Cu") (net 3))
 (segment (start 105.34 88.79) (end 101.975 88.79) (width 1) (layer "F.Cu") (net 3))
 (segment (start 114.9 88.79) (end 114.9 88.61) (width 0.2) (layer "F.Cu") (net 3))
 (segment (start 101.82 88.71) (end 101.9 88.79) (width 1) (layer "F.Cu") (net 3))
 (segment (start 101.82 76.845) (end 101.82 88.71) (width 1) (layer "F.Cu") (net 3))
 (segment (start 123.485 134.51) (end 123.52 134.545) (width 1) (layer "F.Cu") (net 21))
 (segment (start 173.35 81.595) (end 166.585 81.595) (width 1) (layer "F.Cu") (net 21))
 (segment (start 114.735 134.345) (end 114.9 134.51) (width 1) (layer "F.Cu") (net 21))
 (segment (start 188.9 120.98) (end 188.9 111.825) (width 1) (layer "F.Cu") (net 21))
 (segment (start 188.9 111.825) (end 188.9 97.145) (width 1) (layer "F.Cu") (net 21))
 (segment (start 86.865 134.345) (end 114.735 134.345) (width 1) (layer "F.Cu") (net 21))
 (segment (start 181.26 111.825) (end 188.9 111.825) (width 0.7) (layer "F.Cu") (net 21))
 (segment (start 114.9 134.51) (end 123.485 134.51) (width 1) (layer "F.Cu") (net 21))
 (segment (start 178.08 116.675) (end 178.08 115.005) (width 0.7) (layer "F.Cu") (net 21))
 (segment (start 178.08 115.005) (end 181.26 111.825) (width 0.7) (layer "F.Cu") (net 21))
 (segment (start 188.9 97.145) (end 173.35 81.595) (width 1) (layer "F.Cu") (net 21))
 (segment (start 130.89 141.915) (end 167.965 141.915) (width 1) (layer "F.Cu") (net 21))
 (segment (start 167.965 141.915) (end 188.9 120.98) (width 1) (layer "F.Cu") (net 21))
 (segment (start 123.52 134.545) (end 130.89 141.915) (width 1) (layer "F.Cu") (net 21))
 (segment (start 81.8 129.28) (end 86.865 134.345) (width 1) (layer "F.Cu") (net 21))
 (segment (start 75.315 75.075) (end 77.61 75.075) (width 1) (layer "F.Cu") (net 2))
 (segment (start 81.815 79.28) (end 81.815 88.545) (width 1) (layer "F.Cu") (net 2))
 (segment (start 77.61 75.075) (end 81.815 79.28) (width 1) (layer "F.Cu") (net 2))
 (segment (start 157.375 111.685) (end 157.43 111.63) (width 0.7) (layer "F.Cu") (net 29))
 (segment (start 148.92 111.685) (end 157.375 111.685) (width 0.7) (layer "F.Cu") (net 29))
 (segment (start 157.375 132.005) (end 157.43 131.95) (width 0.7) (layer "F.Cu") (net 37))
 (segment (start 148.92 132.005) (end 157.375 132.005) (width 0.7) (layer "F.Cu") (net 37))
 (segment (start 157.375 96.445) (end 157.43 96.39) (width 0.7) (layer "F.Cu") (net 24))
 (segment (start 148.92 96.445) (end 157.375 96.445) (width 0.7) (layer "F.Cu") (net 24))
 (segment (start 148.92 129.465) (end 157.375 129.465) (width 0.7) (layer "F.Cu") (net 36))
 (segment (start 157.375 129.465) (end 157.43 129.41) (width 0.7) (layer "F.Cu") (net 36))
 (segment (start 148.92 121.845) (end 157.375 121.845) (width 0.7) (layer "F.Cu") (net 33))
 (segment (start 157.375 121.845) (end 157.43 121.79) (width 0.7) (layer "F.Cu") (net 33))
 (segment (start 148.92 106.605) (end 157.375 106.605) (width 0.7) (layer "F.Cu") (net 27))
 (segment (start 157.375 106.605) (end 157.43 106.55) (width 0.7) (layer "F.Cu") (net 27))
 (segment (start 148.92 119.305) (end 157.375 119.305) (width 0.7) (layer "F.Cu") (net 32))
 (segment (start 157.375 119.305) (end 157.43 119.25) (width 0.7) (layer "F.Cu") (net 32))
 (segment (start 157.375 134.545) (end 157.43 134.49) (width 0.7) (layer "F.Cu") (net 38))
 (segment (start 148.92 134.545) (end 157.375 134.545) (width 0.7) (layer "F.Cu") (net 38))
 (segment (start 148.92 124.385) (end 157.375 124.385) (width 0.7) (layer "F.Cu") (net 34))
 (segment (start 157.375 124.385) (end 157.43 124.33) (width 0.7) (layer "F.Cu") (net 34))
 (segment (start 157.375 126.925) (end 157.43 126.87) (width 0.7) (layer "F.Cu") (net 35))
 (segment (start 157.43 126.87) (end 161.075 126.87) (width 1) (layer "F.Cu") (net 35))
 (segment (start 148.92 126.925) (end 157.375 126.925) (width 0.7) (layer "F.Cu") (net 35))
 (segment (start 161.075 126.87) (end 164.395 123.55) (width 1) (layer "F.Cu") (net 35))
 (segment (start 157.375 101.525) (end 157.43 101.47) (width 0.7) (layer "F.Cu") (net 26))
 (segment (start 148.92 101.525) (end 157.375 101.525) (width 0.7) (layer "F.Cu") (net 26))
 (segment (start 157.375 98.985) (end 157.43 98.93) (width 0.7) (layer "F.Cu") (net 25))
 (segment (start 148.92 98.985) (end 157.375 98.985) (width 0.7) (layer "F.Cu") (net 25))
 (segment (start 148.92 109.145) (end 157.375 109.145) (width 0.7) (layer "F.Cu") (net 28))
 (segment (start 157.375 109.145) (end 157.43 109.09) (width 0.7) (layer "F.Cu") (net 28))
 (segment (start 123.485 124.35) (end 123.52 124.385) (width 0.7) (layer "F.Cu") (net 17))
 (segment (start 114.9 124.35) (end 123.485 124.35) (width 0.7) (layer "F.Cu") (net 17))
 (segment (start 123.485 101.49) (end 123.52 101.525) (width 0.7) (layer "F.Cu") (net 8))
 (segment (start 114.9 101.49) (end 123.485 101.49) (width 0.7) (layer "F.Cu") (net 8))
 (segment (start 123.485 131.97) (end 123.52 132.005) (width 0.7) (layer "F.Cu") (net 20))
 (segment (start 114.9 131.97) (end 123.485 131.97) (width 0.7) (layer "F.Cu") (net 20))
 (segment (start 114.9 126.89) (end 123.485 126.89) (width 0.7) (layer "F.Cu") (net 18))
 (segment (start 123.485 126.89) (end 123.52 126.925) (width 0.7) (layer "F.Cu") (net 18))
 (segment (start 114.9 93.87) (end 123.485 93.87) (width 0.7) (layer "F.Cu") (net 5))
 (segment (start 123.485 93.87) (end 123.52 93.905) (width 0.7) (layer "F.Cu") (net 5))
 (segment (start 114.9 98.95) (end 123.485 98.95) (width 0.7) (layer "F.Cu") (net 7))
 (segment (start 123.485 98.95) (end 123.52 98.985) (width 0.7) (layer "F.Cu") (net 7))
 (segment (start 114.9 96.41) (end 123.485 96.41) (width 0.7) (layer "F.Cu") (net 6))
 (segment (start 123.485 96.41) (end 123.52 96.445) (width 0.7) (layer "F.Cu") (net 6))
 (segment (start 123.485 119.27) (end 123.52 119.305) (width 0.7) (layer "F.Cu") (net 15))
 (segment (start 114.9 119.27) (end 123.485 119.27) (width 0.7) (layer "F.Cu") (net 15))
 (segment (start 114.9 91.33) (end 123.485 91.33) (width 0.7) (layer "F.Cu") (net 4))
 (segment (start 123.485 91.33) (end 123.52 91.365) (width 0.7) (layer "F.Cu") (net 4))
 (segment (start 123.485 109.11) (end 123.52 109.145) (width 0.7) (layer "F.Cu") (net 11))
 (segment (start 114.9 109.11) (end 123.485 109.11) (width 0.7) (layer "F.Cu") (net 11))
 (segment (start 114.9 116.73) (end 123.485 116.73) (width 0.7) (layer "F.Cu") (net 14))
 (segment (start 123.485 116.73) (end 123.52 116.765) (width 0.7) (layer "F.Cu") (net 14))
 (segment (start 123.485 129.43) (end 123.52 129.465) (width 0.7) (layer "F.Cu") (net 19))
 (segment (start 114.9 129.43) (end 123.485 129.43) (width 0.7) (layer "F.Cu") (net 19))
 (segment (start 89.985 121.765) (end 89.94 121.81) (width 0.7) (layer "F.Cu") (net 16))
 (segment (start 90.025 100.31) (end 89.985 100.35) (width 0.7) (layer "F.Cu") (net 16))
 (segment (start 96.39 73.21) (end 89.985 79.615) (width 0.7) (layer "F.Cu") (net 16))
 (segment (start 102.905 73.21) (end 96.39 73.21) (width 0.7) (layer "F.Cu") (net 16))
 (segment (start 93.495 121.81) (end 97.765 121.81) (width 1) (layer "F.Cu") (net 16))
 (segment (start 157.375 104.065) (end 157.43 104.01) (width 0.7) (layer "F.Cu") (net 16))
 (segment (start 131.14 121.845) (end 147.88 138.585) (width 0.7) (layer "F.Cu") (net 16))
 (segment (start 185.7 119.55) (end 185.7 116.675) (width 0.7) (layer "F.Cu") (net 16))
 (segment (start 148.92 104.065) (end 131.14 121.845) (width 0.7) (layer "F.Cu") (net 16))
 (segment (start 97.765 121.81) (end 103.94 121.81) (width 1) (layer "F.Cu") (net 16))
 (segment (start 147.88 138.585) (end 166.665 138.585) (width 0.7) (layer "F.Cu") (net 16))
 (segment (start 148.92 104.065) (end 157.375 104.065) (width 0.7) (layer "F.Cu") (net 16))
 (segment (start 148.92 88.825) (end 157.375 88.825) (width 0.7) (layer "F.Cu") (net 16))
 (segment (start 170.37 84.135) (end 174.515 88.28) (width 1) (layer "F.Cu") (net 16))
 (segment (start 166.665 138.585) (end 185.7 119.55) (width 0.7) (layer "F.Cu") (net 16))
 (segment (start 168.085 104.045) (end 164.34 104.045) (width 1) (layer "F.Cu") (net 16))
 (segment (start 174.515 97.615) (end 168.085 104.045) (width 1) (layer "F.Cu") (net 16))
 (segment (start 104.36 74.665) (end 102.905 73.21) (width 0.7) (layer "F.Cu") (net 16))
 (segment (start 157.375 88.825) (end 157.43 88.77) (width 0.7) (layer "F.Cu") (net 16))
 (segment (start 131.14 121.845) (end 123.52 121.845) (width 0.7) (layer "F.Cu") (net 16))
 (segment (start 162.065 84.135) (end 157.43 88.77) (width 1) (layer "F.Cu") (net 16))
 (segment (start 93.5 100.31) (end 90.025 100.31) (width 0.7) (layer "F.Cu") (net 16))
 (segment (start 157.465 104.045) (end 157.43 104.01) (width 1) (layer "F.Cu") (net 16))
 (segment (start 123.485 121.81) (end 123.52 121.845) (width 1) (layer "F.Cu") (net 16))
 (segment (start 93.505 121.8) (end 93.495 121.81) (width 1) (layer "F.Cu") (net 16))
 (segment (start 130.875 121.845) (end 123.52 121.845) (width 0.5) (layer "F.Cu") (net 16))
 (segment (start 166.585 84.135) (end 170.37 84.135) (width 1) (layer "F.Cu") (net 16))
 (segment (start 71.17 121.81) (end 89.94 121.81) (width 1) (layer "F.Cu") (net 16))
 (segment (start 89.985 79.615) (end 89.985 100.35) (width 0.7) (layer "F.Cu") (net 16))
 (segment (start 174.515 88.28) (end 174.515 97.615) (width 1) (layer "F.Cu") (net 16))
 (segment (start 91.855 121.81) (end 93.495 121.81) (width 1) (layer "F.Cu") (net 16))
 (segment (start 103.94 121.81) (end 114.9 121.81) (width 1) (layer "F.Cu") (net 16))
 (segment (start 114.935 121.845) (end 114.9 121.81) (width 1) (layer "F.Cu") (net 16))
 (segment (start 63.685 129.295) (end 71.17 121.81) (width 1) (layer "F.Cu") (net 16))
 (segment (start 164.34 104.045) (end 157.465 104.045) (width 1) (layer "F.Cu") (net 16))
 (segment (start 123.52 121.845) (end 114.935 121.845) (width 1) (layer "F.Cu") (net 16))
 (segment (start 89.94 121.81) (end 91.855 121.81) (width 1) (layer "F.Cu") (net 16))
 (segment (start 97.795 121.78) (end 97.765 121.81) (width 0.7) (layer "F.Cu") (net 16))
 (segment (start 104.36 76.845) (end 104.36 74.665) (width 0.7) (layer "F.Cu") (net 16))
 (segment (start 166.585 84.135) (end 162.065 84.135) (width 1) (layer "F.Cu") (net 16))
 (segment (start 89.985 100.35) (end 89.985 121.765) (width 0.7) (layer "F.Cu") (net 16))
 (segment (start 164.395 106.64) (end 164.34 106.585) (width 1) (layer "F.Cu") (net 41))
 (segment (start 164.395 113.39) (end 164.395 106.64) (width 1) (layer "F.Cu") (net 41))
 (segment (start 114.9 104.03) (end 123.485 104.03) (width 0.7) (layer "F.Cu") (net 9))
 (segment (start 123.485 104.03) (end 123.52 104.065) (width 0.7) (layer "F.Cu") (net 9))
 (segment (start 114.9 106.57) (end 123.485 106.57) (width 0.7) (layer "F.Cu") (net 10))
 (segment (start 123.485 106.57) (end 123.52 106.605) (width 0.7) (layer "F.Cu") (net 10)))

